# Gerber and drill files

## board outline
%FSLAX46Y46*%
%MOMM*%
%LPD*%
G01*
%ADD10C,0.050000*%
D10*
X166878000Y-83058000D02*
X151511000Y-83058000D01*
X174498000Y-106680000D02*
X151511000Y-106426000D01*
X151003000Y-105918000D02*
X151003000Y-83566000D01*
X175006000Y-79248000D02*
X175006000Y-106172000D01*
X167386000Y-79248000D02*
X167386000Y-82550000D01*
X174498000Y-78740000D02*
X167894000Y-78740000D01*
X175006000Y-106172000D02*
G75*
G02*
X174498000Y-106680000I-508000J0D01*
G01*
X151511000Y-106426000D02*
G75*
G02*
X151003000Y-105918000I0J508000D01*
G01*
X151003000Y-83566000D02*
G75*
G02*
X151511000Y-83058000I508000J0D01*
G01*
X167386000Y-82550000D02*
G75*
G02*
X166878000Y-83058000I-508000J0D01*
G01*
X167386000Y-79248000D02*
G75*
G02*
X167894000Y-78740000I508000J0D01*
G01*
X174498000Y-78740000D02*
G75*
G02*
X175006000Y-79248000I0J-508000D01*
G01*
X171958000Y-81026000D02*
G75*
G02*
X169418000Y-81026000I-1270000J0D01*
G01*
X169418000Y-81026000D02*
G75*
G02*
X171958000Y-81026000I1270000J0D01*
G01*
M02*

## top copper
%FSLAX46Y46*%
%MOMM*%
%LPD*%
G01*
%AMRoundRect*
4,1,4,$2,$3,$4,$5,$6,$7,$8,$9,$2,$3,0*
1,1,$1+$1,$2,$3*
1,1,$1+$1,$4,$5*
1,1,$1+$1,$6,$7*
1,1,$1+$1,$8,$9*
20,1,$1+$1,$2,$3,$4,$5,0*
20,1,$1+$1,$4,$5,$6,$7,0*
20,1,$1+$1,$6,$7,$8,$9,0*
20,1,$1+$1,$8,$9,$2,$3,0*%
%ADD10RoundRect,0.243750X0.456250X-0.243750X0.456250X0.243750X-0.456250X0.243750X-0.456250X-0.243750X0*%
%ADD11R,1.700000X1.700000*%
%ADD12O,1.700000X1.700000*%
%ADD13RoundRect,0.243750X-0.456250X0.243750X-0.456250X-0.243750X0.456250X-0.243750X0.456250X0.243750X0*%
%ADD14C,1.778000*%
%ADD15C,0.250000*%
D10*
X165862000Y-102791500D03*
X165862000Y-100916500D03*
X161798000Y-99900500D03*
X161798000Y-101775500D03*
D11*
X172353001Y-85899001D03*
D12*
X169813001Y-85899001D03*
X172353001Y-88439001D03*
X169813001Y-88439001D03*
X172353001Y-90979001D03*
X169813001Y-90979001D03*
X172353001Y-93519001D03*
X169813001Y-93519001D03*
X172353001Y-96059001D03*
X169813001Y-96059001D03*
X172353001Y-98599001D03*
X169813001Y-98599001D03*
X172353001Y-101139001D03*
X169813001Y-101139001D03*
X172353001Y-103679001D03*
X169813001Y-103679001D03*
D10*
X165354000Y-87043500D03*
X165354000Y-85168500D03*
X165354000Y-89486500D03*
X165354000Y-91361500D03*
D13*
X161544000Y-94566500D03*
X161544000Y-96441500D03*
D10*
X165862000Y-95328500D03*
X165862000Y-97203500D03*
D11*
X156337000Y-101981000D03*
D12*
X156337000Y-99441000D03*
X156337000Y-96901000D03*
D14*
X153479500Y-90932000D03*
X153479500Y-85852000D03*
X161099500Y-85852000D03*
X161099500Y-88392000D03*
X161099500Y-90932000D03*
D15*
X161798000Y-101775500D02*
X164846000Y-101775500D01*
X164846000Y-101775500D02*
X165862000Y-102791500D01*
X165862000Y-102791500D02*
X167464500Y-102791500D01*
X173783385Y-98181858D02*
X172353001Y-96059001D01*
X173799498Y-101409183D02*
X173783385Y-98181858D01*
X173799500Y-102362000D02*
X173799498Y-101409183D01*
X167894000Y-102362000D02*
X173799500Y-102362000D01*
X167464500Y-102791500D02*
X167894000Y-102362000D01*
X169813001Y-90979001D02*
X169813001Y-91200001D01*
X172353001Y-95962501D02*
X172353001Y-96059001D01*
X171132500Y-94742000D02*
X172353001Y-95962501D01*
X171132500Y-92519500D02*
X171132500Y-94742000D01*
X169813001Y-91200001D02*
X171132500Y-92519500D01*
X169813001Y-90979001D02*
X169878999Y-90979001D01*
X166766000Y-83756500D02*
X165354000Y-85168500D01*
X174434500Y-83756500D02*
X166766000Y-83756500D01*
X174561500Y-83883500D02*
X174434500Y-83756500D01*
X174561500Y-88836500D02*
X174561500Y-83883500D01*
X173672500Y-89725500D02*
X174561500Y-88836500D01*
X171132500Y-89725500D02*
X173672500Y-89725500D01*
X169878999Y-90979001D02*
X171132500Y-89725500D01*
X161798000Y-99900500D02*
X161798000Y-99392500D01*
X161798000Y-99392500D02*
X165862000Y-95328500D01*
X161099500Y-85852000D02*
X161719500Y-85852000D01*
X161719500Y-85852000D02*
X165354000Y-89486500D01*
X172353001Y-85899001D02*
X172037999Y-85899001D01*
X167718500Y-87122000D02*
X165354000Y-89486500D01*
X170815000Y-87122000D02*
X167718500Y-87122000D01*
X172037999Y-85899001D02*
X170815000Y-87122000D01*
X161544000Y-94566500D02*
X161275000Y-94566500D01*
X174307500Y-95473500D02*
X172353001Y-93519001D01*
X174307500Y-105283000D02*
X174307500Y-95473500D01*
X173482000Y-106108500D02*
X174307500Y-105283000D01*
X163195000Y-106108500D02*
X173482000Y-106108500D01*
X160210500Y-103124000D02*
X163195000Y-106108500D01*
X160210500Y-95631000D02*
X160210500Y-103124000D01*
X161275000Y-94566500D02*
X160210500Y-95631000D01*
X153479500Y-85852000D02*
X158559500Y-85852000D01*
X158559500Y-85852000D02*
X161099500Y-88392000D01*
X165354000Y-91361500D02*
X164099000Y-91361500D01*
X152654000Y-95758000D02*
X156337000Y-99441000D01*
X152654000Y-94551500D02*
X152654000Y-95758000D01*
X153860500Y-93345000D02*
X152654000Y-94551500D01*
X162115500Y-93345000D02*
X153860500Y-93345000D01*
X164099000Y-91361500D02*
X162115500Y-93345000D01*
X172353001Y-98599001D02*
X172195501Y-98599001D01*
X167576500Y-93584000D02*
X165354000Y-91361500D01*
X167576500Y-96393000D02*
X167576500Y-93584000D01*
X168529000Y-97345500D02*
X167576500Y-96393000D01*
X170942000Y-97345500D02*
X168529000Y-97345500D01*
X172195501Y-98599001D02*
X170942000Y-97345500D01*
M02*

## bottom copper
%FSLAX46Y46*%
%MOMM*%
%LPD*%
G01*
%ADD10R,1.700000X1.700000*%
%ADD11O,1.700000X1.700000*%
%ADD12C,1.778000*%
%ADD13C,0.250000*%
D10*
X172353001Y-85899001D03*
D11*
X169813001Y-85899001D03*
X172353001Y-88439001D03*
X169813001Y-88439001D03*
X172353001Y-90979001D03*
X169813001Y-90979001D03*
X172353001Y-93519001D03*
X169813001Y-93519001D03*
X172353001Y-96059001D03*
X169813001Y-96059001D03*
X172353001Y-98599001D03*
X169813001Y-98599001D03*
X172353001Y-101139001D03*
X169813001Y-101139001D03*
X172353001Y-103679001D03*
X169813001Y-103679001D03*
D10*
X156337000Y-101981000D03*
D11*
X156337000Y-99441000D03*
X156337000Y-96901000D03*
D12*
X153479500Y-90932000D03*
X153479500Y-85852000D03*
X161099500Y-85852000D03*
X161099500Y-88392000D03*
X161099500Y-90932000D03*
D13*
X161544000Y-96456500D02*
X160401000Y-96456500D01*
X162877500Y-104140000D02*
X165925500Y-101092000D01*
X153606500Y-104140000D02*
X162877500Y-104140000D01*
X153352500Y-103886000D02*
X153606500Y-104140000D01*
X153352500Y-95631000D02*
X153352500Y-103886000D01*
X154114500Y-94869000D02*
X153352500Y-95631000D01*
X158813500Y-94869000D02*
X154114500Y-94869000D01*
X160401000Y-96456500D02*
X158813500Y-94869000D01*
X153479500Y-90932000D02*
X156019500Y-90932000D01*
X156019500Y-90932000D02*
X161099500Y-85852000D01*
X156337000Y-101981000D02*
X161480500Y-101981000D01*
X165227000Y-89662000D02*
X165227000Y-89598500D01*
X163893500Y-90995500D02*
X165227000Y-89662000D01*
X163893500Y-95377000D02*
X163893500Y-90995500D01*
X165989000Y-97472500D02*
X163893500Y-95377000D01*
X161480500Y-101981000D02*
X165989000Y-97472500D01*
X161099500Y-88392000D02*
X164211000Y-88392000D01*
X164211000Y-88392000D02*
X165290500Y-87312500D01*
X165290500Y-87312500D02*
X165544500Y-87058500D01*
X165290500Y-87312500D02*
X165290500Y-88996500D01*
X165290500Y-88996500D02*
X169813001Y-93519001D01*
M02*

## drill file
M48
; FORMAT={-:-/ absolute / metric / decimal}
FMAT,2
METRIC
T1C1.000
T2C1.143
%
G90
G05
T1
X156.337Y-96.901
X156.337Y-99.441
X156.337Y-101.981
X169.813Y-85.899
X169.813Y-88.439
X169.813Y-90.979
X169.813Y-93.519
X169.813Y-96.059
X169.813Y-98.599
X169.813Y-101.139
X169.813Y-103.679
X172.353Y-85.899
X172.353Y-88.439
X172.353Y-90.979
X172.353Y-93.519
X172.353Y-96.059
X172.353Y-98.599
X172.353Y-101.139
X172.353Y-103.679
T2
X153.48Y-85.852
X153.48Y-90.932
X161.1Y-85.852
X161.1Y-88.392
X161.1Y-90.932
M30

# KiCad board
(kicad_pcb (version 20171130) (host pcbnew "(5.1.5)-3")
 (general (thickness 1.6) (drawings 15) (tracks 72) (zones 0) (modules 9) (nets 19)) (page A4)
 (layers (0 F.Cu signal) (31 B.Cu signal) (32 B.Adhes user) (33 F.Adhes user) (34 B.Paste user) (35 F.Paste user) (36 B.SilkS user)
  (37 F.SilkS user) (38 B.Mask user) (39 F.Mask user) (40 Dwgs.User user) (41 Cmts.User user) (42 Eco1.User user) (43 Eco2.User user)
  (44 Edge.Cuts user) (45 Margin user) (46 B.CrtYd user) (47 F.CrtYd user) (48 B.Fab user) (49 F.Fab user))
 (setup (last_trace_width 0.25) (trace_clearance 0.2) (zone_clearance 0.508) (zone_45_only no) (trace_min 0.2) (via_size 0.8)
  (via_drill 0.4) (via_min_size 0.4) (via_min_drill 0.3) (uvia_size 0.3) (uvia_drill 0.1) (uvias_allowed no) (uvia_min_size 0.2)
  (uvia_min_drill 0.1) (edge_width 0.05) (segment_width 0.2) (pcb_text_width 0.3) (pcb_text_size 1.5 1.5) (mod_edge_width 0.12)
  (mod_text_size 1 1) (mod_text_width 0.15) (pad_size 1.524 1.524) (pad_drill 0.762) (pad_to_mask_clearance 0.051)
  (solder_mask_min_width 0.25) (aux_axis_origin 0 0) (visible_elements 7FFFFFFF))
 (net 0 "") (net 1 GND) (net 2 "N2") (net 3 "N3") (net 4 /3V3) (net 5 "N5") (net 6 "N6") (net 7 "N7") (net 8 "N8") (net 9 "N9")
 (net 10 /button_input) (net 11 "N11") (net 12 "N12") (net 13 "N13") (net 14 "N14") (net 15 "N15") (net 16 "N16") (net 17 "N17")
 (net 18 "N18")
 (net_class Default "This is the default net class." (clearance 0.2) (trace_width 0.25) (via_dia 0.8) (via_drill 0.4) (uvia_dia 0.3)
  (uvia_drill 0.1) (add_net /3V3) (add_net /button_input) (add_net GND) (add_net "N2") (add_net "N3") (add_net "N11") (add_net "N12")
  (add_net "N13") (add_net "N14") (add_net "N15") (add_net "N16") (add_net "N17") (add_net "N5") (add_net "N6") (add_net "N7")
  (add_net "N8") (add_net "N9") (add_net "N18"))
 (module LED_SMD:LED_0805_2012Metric (layer F.Cu) (at 165.862 101.854 90)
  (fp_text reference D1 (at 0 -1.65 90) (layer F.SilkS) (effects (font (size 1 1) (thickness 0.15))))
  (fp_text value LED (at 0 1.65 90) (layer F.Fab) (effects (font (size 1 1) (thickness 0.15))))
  (pad 1 smd roundrect (at -0.9375 0 90) (size 0.975 1.4) (layers F.Cu F.Paste F.Mask) (roundrect_rratio 0.25) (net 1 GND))
  (pad 2 smd roundrect (at 0.9375 0 90) (size 0.975 1.4) (layers F.Cu F.Paste F.Mask) (roundrect_rratio 0.25) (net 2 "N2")))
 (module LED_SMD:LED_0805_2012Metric (layer F.Cu) (at 161.798 100.838 90)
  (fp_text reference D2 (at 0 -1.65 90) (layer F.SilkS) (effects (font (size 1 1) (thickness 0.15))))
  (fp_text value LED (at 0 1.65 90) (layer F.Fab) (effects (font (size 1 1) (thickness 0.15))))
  (pad 2 smd roundrect (at 0.9375 0 90) (size 0.975 1.4) (layers F.Cu F.Paste F.Mask) (roundrect_rratio 0.25) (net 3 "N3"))
  (pad 1 smd roundrect (at -0.9375 0 90) (size 0.975 1.4) (layers F.Cu F.Paste F.Mask) (roundrect_rratio 0.25) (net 1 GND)))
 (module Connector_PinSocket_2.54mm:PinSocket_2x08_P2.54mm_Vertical (layer F.Cu) (at 172.353001 85.899001)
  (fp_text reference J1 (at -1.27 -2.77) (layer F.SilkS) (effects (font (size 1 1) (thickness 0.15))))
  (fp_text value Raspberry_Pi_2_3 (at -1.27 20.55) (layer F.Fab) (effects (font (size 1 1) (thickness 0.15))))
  (pad 1 thru_hole rect (at 0 0) (size 1.7 1.7) (drill 1) (layers *.Cu *.Mask) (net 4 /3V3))
  (pad 2 thru_hole oval (at -2.54 0) (size 1.7 1.7) (drill 1) (layers *.Cu *.Mask) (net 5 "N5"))
  (pad 3 thru_hole oval (at 0 2.54) (size 1.7 1.7) (drill 1) (layers *.Cu *.Mask) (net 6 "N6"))
  (pad 4 thru_hole oval (at -2.54 2.54) (size 1.7 1.7) (drill 1) (layers *.Cu *.Mask) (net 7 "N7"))
  (pad 5 thru_hole oval (at 0 5.08) (size 1.7 1.7) (drill 1) (layers *.Cu *.Mask) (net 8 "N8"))
  (pad 6 thru_hole oval (at -2.54 5.08) (size 1.7 1.7) (drill 1) (layers *.Cu *.Mask) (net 1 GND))
  (pad 7 thru_hole oval (at 0 7.62) (size 1.7 1.7) (drill 1) (layers *.Cu *.Mask) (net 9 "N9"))
  (pad 8 thru_hole oval (at -2.54 7.62) (size 1.7 1.7) (drill 1) (layers *.Cu *.Mask) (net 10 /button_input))
  (pad 9 thru_hole oval (at 0 10.16) (size 1.7 1.7) (drill 1) (layers *.Cu *.Mask) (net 1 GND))
  (pad 10 thru_hole oval (at -2.54 10.16) (size 1.7 1.7) (drill 1) (layers *.Cu *.Mask) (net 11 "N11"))
  (pad 11 thru_hole oval (at 0 12.7) (size 1.7 1.7) (drill 1) (layers *.Cu *.Mask) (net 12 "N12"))
  (pad 12 thru_hole oval (at -2.54 12.7) (size 1.7 1.7) (drill 1) (layers *.Cu *.Mask) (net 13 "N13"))
  (pad 13 thru_hole oval (at 0 15.24) (size 1.7 1.7) (drill 1) (layers *.Cu *.Mask) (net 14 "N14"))
  (pad 14 thru_hole oval (at -2.54 15.24) (size 1.7 1.7) (drill 1) (layers *.Cu *.Mask) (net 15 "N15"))
  (pad 15 thru_hole oval (at 0 17.78) (size 1.7 1.7) (drill 1) (layers *.Cu *.Mask) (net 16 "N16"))
  (pad 16 thru_hole oval (at -2.54 17.78) (size 1.7 1.7) (drill 1) (layers *.Cu *.Mask) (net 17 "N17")))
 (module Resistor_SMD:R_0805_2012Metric (layer F.Cu) (at 165.354 86.106 90)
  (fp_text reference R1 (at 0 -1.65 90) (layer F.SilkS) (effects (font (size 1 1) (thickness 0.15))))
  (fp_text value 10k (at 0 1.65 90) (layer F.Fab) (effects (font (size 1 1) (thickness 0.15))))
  (pad 1 smd roundrect (at -0.9375 0 90) (size 0.975 1.4) (layers F.Cu F.Paste F.Mask) (roundrect_rratio 0.25) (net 10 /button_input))
  (pad 2 smd roundrect (at 0.9375 0 90) (size 0.975 1.4) (layers F.Cu F.Paste F.Mask) (roundrect_rratio 0.25) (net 1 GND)))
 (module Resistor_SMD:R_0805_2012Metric (layer F.Cu) (at 165.354 90.424 90)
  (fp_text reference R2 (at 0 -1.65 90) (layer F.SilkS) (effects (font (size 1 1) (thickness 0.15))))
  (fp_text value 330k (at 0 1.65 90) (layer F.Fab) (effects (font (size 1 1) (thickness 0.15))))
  (pad 2 smd roundrect (at 0.9375 0 90) (size 0.975 1.4) (layers F.Cu F.Paste F.Mask) (roundrect_rratio 0.25) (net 4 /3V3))
  (pad 1 smd roundrect (at -0.9375 0 90) (size 0.975 1.4) (layers F.Cu F.Paste F.Mask) (roundrect_rratio 0.25) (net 12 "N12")))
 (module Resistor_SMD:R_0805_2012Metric (layer F.Cu) (at 161.544 95.504 270)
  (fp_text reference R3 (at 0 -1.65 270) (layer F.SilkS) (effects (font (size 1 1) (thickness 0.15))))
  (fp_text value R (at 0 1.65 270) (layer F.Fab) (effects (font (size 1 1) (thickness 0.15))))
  (pad 1 smd roundrect (at -0.9375 0 270) (size 0.975 1.4) (layers F.Cu F.Paste F.Mask) (roundrect_rratio 0.25) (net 9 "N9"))
  (pad 2 smd roundrect (at 0.9375 0 270) (size 0.975 1.4) (layers F.Cu F.Paste F.Mask) (roundrect_rratio 0.25) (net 2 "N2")))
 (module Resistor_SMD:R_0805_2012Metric (layer F.Cu) (at 165.862 96.266 90)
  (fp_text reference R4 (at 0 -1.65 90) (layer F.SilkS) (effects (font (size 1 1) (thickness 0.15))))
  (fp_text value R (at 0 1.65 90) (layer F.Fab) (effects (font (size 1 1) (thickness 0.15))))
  (pad 2 smd roundrect (at 0.9375 0 90) (size 0.975 1.4) (layers F.Cu F.Paste F.Mask) (roundrect_rratio 0.25) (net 3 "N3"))
  (pad 1 smd roundrect (at -0.9375 0 90) (size 0.975 1.4) (layers F.Cu F.Paste F.Mask) (roundrect_rratio 0.25) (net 4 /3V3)))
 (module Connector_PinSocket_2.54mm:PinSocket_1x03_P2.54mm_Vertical (layer F.Cu) (at 156.337 101.981 180)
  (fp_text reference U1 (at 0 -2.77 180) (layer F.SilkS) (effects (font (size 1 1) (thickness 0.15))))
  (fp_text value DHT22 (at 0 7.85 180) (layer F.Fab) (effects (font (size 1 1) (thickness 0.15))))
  (pad 1 thru_hole rect (at 0 0 180) (size 1.7 1.7) (drill 1) (layers *.Cu *.Mask) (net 4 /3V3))
  (pad 2 thru_hole oval (at 0 2.54 180) (size 1.7 1.7) (drill 1) (layers *.Cu *.Mask) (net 12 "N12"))
  (pad 3 thru_hole oval (at 0 5.08 180) (size 1.7 1.7) (drill 1) (layers *.Cu *.Mask) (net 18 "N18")))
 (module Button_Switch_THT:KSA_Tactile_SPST (layer F.Cu) (at 153.4795 90.932 90)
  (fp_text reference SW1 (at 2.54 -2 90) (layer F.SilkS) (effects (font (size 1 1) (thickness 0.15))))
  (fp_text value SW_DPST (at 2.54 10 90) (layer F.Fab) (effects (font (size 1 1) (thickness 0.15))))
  (pad 1 thru_hole circle (at 0 0 90) (size 1.778 1.778) (drill 1.143) (layers *.Cu *.Mask) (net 4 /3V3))
  (pad 2 thru_hole circle (at 5.08 0 90) (size 1.778 1.778) (drill 1.143) (layers *.Cu *.Mask) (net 10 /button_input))
  (pad 3 thru_hole circle (at 5.08 7.62 90) (size 1.778 1.778) (drill 1.143) (layers *.Cu *.Mask) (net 4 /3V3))
  (pad 4 thru_hole circle (at 2.54 7.62 90) (size 1.778 1.778) (drill 1.143) (layers *.Cu *.Mask) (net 10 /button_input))
  (pad 5 thru_hole circle (at 0 7.62 90) (size 1.778 1.778) (drill 1.143) (layers *.Cu *.Mask)))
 (gr_line (start 166.878 83.058) (end 151.511 83.058) (angle 90) (layer Edge.Cuts) (width 0.05))
 (gr_line (start 174.498 106.68) (end 151.511 106.426) (angle 90) (layer Edge.Cuts) (width 0.05))
 (gr_line (start 151.003 105.918) (end 151.003 83.566) (angle 90) (layer Edge.Cuts) (width 0.05))
 (gr_line (start 175.006 79.248) (end 175.006 106.172) (angle 90) (layer Edge.Cuts) (width 0.05))
 (gr_line (start 167.386 79.248) (end 167.386 82.55) (angle 90) (layer Edge.Cuts) (width 0.05))
 (gr_line (start 174.498 78.74) (end 167.894 78.74) (angle 90) (layer Edge.Cuts) (width 0.05))
 (gr_arc (start 174.498 106.172) (end 175.006 106.172) (angle 90) (layer Edge.Cuts) (width 0.05))
 (gr_arc (start 151.511 105.918) (end 151.511 106.426) (angle 90) (layer Edge.Cuts) (width 0.05))
 (gr_arc (start 151.511 83.566) (end 151.003 83.566) (angle 90) (layer Edge.Cuts) (width 0.05))
 (gr_arc (start 166.878 82.55) (end 167.386 82.55) (angle 90) (layer Edge.Cuts) (width 0.05))
 (gr_arc (start 167.894 79.248) (end 167.386 79.248) (angle 90) (layer Edge.Cuts) (width 0.05))
 (gr_arc (start 174.498 79.248) (end 174.498 78.74) (angle 90) (layer Edge.Cuts) (width 0.05))
 (gr_circle (center 170.688 81.026) (end 171.704 81.788) (layer Edge.Cuts) (width 0.05))
 (segment (start 161.544 96.4565) (end 160.401 96.4565) (width 0.25) (layer B.Cu) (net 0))
 (segment (start 162.8775 104.14) (end 165.9255 101.092) (width 0.25) (layer B.Cu) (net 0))
 (segment (start 153.6065 104.14) (end 162.8775 104.14) (width 0.25) (layer B.Cu) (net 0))
 (segment (start 153.3525 103.886) (end 153.6065 104.14) (width 0.25) (layer B.Cu) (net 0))
 (segment (start 153.3525 95.631) (end 153.3525 103.886) (width 0.25) (layer B.Cu) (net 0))
 (segment (start 154.1145 94.869) (end 153.3525 95.631) (width 0.25) (layer B.Cu) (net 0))
 (segment (start 158.8135 94.869) (end 154.1145 94.869) (width 0.25) (layer B.Cu) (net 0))
 (segment (start 160.401 96.4565) (end 158.8135 94.869) (width 0.25) (layer B.Cu) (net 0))
 (segment (start 161.798 101.7755) (end 164.846 101.7755) (width 0.25) (layer F.Cu) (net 1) (status 400000))
 (segment (start 164.846 101.7755) (end 165.862 102.7915) (width 0.25) (layer F.Cu) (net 1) (status 800000))
 (segment (start 165.862 102.7915) (end 167.4645 102.7915) (width 0.25) (layer F.Cu) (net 1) (status 400000))
 (segment (start 173.783385 98.181858) (end 172.353001 96.059001) (width 0.25) (layer F.Cu) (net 1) (status 800000))
 (segment (start 173.799498 101.409183) (end 173.783385 98.181858) (width 0.25) (layer F.Cu) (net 1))
 (segment (start 173.7995 102.362) (end 173.799498 101.409183) (width 0.25) (layer F.Cu) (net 1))
 (segment (start 167.894 102.362) (end 173.7995 102.362) (width 0.25) (layer F.Cu) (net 1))
 (segment (start 167.4645 102.7915) (end 167.894 102.362) (width 0.25) (layer F.Cu) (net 1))
 (segment (start 169.813001 90.979001) (end 169.813001 91.200001) (width 0.25) (layer F.Cu) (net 1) (status C00000))
 (segment (start 172.353001 95.962501) (end 172.353001 96.059001) (width 0.25) (layer F.Cu) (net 1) (status C00000))
 (segment (start 171.1325 94.742) (end 172.353001 95.962501) (width 0.25) (layer F.Cu) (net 1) (status 800000))
 (segment (start 171.1325 92.5195) (end 171.1325 94.742) (width 0.25) (layer F.Cu) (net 1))
 (segment (start 169.813001 91.200001) (end 171.1325 92.5195) (width 0.25) (layer F.Cu) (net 1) (status 400000))
 (segment (start 169.813001 90.979001) (end 169.878999 90.979001) (width 0.25) (layer F.Cu) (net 1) (status C00000))
 (segment (start 166.766 83.7565) (end 165.354 85.1685) (width 0.25) (layer F.Cu) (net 1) (status 800000))
 (segment (start 174.4345 83.7565) (end 166.766 83.7565) (width 0.25) (layer F.Cu) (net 1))
 (segment (start 174.5615 83.8835) (end 174.4345 83.7565) (width 0.25) (layer F.Cu) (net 1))
 (segment (start 174.5615 88.8365) (end 174.5615 83.8835) (width 0.25) (layer F.Cu) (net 1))
 (segment (start 173.6725 89.7255) (end 174.5615 88.8365) (width 0.25) (layer F.Cu) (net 1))
 (segment (start 171.1325 89.7255) (end 173.6725 89.7255) (width 0.25) (layer F.Cu) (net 1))
 (segment (start 169.878999 90.979001) (end 171.1325 89.7255) (width 0.25) (layer F.Cu) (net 1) (status 400000))
 (segment (start 161.798 99.9005) (end 161.798 99.3925) (width 0.25) (layer F.Cu) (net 3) (status 400000))
 (segment (start 161.798 99.3925) (end 165.862 95.3285) (width 0.25) (layer F.Cu) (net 3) (status 800000))
 (segment (start 161.0995 85.852) (end 161.7195 85.852) (width 0.25) (layer F.Cu) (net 4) (status C00000))
 (segment (start 161.7195 85.852) (end 165.354 89.4865) (width 0.25) (layer F.Cu) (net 4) (status C00000))
 (segment (start 172.353001 85.899001) (end 172.037999 85.899001) (width 0.25) (layer F.Cu) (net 4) (status C00000))
 (segment (start 167.7185 87.122) (end 165.354 89.4865) (width 0.25) (layer F.Cu) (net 4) (status 800000))
 (segment (start 170.815 87.122) (end 167.7185 87.122) (width 0.25) (layer F.Cu) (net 4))
 (segment (start 172.037999 85.899001) (end 170.815 87.122) (width 0.25) (layer F.Cu) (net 4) (status 400000))
 (segment (start 153.4795 90.932) (end 156.0195 90.932) (width 0.25) (layer B.Cu) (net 4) (status 400000))
 (segment (start 156.0195 90.932) (end 161.0995 85.852) (width 0.25) (layer B.Cu) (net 4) (status 800000))
 (segment (start 156.337 101.981) (end 161.4805 101.981) (width 0.25) (layer B.Cu) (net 4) (status 400000))
 (segment (start 165.227 89.662) (end 165.227 89.5985) (width 0.25) (layer B.Cu) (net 4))
 (segment (start 163.8935 90.9955) (end 165.227 89.662) (width 0.25) (layer B.Cu) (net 4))
 (segment (start 163.8935 95.377) (end 163.8935 90.9955) (width 0.25) (layer B.Cu) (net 4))
 (segment (start 165.989 97.4725) (end 163.8935 95.377) (width 0.25) (layer B.Cu) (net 4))
 (segment (start 161.4805 101.981) (end 165.989 97.4725) (width 0.25) (layer B.Cu) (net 4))
 (segment (start 161.544 94.5665) (end 161.275 94.5665) (width 0.25) (layer F.Cu) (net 9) (status C00000))
 (segment (start 174.3075 95.4735) (end 172.353001 93.519001) (width 0.25) (layer F.Cu) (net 9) (status 800000))
 (segment (start 174.3075 105.283) (end 174.3075 95.4735) (width 0.25) (layer F.Cu) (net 9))
 (segment (start 173.482 106.1085) (end 174.3075 105.283) (width 0.25) (layer F.Cu) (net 9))
 (segment (start 163.195 106.1085) (end 173.482 106.1085) (width 0.25) (layer F.Cu) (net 9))
 (segment (start 160.2105 103.124) (end 163.195 106.1085) (width 0.25) (layer F.Cu) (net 9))
 (segment (start 160.2105 95.631) (end 160.2105 103.124) (width 0.25) (layer F.Cu) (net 9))
 (segment (start 161.275 94.5665) (end 160.2105 95.631) (width 0.25) (layer F.Cu) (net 9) (status 400000))
 (segment (start 153.4795 85.852) (end 158.5595 85.852) (width 0.25) (layer F.Cu) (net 10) (status 400000))
 (segment (start 158.5595 85.852) (end 161.0995 88.392) (width 0.25) (layer F.Cu) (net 10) (status 800000))
 (segment (start 161.0995 88.392) (end 164.211 88.392) (width 0.25) (layer B.Cu) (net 10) (status 400000))
 (segment (start 164.211 88.392) (end 165.2905 87.3125) (width 0.25) (layer B.Cu) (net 10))
 (segment (start 165.2905 87.3125) (end 165.5445 87.0585) (width 0.25) (layer B.Cu) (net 10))
 (segment (start 165.2905 87.3125) (end 165.2905 88.9965) (width 0.25) (layer B.Cu) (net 10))
 (segment (start 165.2905 88.9965) (end 169.813001 93.519001) (width 0.25) (layer B.Cu) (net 10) (status 800000))
 (segment (start 165.354 91.3615) (end 164.099 91.3615) (width 0.25) (layer F.Cu) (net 12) (status 400000))
 (segment (start 152.654 95.758) (end 156.337 99.441) (width 0.25) (layer F.Cu) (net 12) (status 800000))
 (segment (start 152.654 94.5515) (end 152.654 95.758) (width 0.25) (layer F.Cu) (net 12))
 (segment (start 153.8605 93.345) (end 152.654 94.5515) (width 0.25) (layer F.Cu) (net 12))
 (segment (start 162.1155 93.345) (end 153.8605 93.345) (width 0.25) (layer F.Cu) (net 12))
 (segment (start 164.099 91.3615) (end 162.1155 93.345) (width 0.25) (layer F.Cu) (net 12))
 (segment (start 172.353001 98.599001) (end 172.195501 98.599001) (width 0.25) (layer F.Cu) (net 12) (status C00000))
 (segment (start 167.5765 93.584) (end 165.354 91.3615) (width 0.25) (layer F.Cu) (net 12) (status 800000))
 (segment (start 167.5765 96.393) (end 167.5765 93.584) (width 0.25) (layer F.Cu) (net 12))
 (segment (start 168.529 97.3455) (end 167.5765 96.393) (width 0.25) (layer F.Cu) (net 12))
 (segment (start 170.942 97.3455) (end 168.529 97.3455) (width 0.25) (layer F.Cu) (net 12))
 (segment (start 172.195501 98.599001) (end 170.942 97.3455) (width 0.25) (layer F.Cu) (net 12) (status 400000)))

